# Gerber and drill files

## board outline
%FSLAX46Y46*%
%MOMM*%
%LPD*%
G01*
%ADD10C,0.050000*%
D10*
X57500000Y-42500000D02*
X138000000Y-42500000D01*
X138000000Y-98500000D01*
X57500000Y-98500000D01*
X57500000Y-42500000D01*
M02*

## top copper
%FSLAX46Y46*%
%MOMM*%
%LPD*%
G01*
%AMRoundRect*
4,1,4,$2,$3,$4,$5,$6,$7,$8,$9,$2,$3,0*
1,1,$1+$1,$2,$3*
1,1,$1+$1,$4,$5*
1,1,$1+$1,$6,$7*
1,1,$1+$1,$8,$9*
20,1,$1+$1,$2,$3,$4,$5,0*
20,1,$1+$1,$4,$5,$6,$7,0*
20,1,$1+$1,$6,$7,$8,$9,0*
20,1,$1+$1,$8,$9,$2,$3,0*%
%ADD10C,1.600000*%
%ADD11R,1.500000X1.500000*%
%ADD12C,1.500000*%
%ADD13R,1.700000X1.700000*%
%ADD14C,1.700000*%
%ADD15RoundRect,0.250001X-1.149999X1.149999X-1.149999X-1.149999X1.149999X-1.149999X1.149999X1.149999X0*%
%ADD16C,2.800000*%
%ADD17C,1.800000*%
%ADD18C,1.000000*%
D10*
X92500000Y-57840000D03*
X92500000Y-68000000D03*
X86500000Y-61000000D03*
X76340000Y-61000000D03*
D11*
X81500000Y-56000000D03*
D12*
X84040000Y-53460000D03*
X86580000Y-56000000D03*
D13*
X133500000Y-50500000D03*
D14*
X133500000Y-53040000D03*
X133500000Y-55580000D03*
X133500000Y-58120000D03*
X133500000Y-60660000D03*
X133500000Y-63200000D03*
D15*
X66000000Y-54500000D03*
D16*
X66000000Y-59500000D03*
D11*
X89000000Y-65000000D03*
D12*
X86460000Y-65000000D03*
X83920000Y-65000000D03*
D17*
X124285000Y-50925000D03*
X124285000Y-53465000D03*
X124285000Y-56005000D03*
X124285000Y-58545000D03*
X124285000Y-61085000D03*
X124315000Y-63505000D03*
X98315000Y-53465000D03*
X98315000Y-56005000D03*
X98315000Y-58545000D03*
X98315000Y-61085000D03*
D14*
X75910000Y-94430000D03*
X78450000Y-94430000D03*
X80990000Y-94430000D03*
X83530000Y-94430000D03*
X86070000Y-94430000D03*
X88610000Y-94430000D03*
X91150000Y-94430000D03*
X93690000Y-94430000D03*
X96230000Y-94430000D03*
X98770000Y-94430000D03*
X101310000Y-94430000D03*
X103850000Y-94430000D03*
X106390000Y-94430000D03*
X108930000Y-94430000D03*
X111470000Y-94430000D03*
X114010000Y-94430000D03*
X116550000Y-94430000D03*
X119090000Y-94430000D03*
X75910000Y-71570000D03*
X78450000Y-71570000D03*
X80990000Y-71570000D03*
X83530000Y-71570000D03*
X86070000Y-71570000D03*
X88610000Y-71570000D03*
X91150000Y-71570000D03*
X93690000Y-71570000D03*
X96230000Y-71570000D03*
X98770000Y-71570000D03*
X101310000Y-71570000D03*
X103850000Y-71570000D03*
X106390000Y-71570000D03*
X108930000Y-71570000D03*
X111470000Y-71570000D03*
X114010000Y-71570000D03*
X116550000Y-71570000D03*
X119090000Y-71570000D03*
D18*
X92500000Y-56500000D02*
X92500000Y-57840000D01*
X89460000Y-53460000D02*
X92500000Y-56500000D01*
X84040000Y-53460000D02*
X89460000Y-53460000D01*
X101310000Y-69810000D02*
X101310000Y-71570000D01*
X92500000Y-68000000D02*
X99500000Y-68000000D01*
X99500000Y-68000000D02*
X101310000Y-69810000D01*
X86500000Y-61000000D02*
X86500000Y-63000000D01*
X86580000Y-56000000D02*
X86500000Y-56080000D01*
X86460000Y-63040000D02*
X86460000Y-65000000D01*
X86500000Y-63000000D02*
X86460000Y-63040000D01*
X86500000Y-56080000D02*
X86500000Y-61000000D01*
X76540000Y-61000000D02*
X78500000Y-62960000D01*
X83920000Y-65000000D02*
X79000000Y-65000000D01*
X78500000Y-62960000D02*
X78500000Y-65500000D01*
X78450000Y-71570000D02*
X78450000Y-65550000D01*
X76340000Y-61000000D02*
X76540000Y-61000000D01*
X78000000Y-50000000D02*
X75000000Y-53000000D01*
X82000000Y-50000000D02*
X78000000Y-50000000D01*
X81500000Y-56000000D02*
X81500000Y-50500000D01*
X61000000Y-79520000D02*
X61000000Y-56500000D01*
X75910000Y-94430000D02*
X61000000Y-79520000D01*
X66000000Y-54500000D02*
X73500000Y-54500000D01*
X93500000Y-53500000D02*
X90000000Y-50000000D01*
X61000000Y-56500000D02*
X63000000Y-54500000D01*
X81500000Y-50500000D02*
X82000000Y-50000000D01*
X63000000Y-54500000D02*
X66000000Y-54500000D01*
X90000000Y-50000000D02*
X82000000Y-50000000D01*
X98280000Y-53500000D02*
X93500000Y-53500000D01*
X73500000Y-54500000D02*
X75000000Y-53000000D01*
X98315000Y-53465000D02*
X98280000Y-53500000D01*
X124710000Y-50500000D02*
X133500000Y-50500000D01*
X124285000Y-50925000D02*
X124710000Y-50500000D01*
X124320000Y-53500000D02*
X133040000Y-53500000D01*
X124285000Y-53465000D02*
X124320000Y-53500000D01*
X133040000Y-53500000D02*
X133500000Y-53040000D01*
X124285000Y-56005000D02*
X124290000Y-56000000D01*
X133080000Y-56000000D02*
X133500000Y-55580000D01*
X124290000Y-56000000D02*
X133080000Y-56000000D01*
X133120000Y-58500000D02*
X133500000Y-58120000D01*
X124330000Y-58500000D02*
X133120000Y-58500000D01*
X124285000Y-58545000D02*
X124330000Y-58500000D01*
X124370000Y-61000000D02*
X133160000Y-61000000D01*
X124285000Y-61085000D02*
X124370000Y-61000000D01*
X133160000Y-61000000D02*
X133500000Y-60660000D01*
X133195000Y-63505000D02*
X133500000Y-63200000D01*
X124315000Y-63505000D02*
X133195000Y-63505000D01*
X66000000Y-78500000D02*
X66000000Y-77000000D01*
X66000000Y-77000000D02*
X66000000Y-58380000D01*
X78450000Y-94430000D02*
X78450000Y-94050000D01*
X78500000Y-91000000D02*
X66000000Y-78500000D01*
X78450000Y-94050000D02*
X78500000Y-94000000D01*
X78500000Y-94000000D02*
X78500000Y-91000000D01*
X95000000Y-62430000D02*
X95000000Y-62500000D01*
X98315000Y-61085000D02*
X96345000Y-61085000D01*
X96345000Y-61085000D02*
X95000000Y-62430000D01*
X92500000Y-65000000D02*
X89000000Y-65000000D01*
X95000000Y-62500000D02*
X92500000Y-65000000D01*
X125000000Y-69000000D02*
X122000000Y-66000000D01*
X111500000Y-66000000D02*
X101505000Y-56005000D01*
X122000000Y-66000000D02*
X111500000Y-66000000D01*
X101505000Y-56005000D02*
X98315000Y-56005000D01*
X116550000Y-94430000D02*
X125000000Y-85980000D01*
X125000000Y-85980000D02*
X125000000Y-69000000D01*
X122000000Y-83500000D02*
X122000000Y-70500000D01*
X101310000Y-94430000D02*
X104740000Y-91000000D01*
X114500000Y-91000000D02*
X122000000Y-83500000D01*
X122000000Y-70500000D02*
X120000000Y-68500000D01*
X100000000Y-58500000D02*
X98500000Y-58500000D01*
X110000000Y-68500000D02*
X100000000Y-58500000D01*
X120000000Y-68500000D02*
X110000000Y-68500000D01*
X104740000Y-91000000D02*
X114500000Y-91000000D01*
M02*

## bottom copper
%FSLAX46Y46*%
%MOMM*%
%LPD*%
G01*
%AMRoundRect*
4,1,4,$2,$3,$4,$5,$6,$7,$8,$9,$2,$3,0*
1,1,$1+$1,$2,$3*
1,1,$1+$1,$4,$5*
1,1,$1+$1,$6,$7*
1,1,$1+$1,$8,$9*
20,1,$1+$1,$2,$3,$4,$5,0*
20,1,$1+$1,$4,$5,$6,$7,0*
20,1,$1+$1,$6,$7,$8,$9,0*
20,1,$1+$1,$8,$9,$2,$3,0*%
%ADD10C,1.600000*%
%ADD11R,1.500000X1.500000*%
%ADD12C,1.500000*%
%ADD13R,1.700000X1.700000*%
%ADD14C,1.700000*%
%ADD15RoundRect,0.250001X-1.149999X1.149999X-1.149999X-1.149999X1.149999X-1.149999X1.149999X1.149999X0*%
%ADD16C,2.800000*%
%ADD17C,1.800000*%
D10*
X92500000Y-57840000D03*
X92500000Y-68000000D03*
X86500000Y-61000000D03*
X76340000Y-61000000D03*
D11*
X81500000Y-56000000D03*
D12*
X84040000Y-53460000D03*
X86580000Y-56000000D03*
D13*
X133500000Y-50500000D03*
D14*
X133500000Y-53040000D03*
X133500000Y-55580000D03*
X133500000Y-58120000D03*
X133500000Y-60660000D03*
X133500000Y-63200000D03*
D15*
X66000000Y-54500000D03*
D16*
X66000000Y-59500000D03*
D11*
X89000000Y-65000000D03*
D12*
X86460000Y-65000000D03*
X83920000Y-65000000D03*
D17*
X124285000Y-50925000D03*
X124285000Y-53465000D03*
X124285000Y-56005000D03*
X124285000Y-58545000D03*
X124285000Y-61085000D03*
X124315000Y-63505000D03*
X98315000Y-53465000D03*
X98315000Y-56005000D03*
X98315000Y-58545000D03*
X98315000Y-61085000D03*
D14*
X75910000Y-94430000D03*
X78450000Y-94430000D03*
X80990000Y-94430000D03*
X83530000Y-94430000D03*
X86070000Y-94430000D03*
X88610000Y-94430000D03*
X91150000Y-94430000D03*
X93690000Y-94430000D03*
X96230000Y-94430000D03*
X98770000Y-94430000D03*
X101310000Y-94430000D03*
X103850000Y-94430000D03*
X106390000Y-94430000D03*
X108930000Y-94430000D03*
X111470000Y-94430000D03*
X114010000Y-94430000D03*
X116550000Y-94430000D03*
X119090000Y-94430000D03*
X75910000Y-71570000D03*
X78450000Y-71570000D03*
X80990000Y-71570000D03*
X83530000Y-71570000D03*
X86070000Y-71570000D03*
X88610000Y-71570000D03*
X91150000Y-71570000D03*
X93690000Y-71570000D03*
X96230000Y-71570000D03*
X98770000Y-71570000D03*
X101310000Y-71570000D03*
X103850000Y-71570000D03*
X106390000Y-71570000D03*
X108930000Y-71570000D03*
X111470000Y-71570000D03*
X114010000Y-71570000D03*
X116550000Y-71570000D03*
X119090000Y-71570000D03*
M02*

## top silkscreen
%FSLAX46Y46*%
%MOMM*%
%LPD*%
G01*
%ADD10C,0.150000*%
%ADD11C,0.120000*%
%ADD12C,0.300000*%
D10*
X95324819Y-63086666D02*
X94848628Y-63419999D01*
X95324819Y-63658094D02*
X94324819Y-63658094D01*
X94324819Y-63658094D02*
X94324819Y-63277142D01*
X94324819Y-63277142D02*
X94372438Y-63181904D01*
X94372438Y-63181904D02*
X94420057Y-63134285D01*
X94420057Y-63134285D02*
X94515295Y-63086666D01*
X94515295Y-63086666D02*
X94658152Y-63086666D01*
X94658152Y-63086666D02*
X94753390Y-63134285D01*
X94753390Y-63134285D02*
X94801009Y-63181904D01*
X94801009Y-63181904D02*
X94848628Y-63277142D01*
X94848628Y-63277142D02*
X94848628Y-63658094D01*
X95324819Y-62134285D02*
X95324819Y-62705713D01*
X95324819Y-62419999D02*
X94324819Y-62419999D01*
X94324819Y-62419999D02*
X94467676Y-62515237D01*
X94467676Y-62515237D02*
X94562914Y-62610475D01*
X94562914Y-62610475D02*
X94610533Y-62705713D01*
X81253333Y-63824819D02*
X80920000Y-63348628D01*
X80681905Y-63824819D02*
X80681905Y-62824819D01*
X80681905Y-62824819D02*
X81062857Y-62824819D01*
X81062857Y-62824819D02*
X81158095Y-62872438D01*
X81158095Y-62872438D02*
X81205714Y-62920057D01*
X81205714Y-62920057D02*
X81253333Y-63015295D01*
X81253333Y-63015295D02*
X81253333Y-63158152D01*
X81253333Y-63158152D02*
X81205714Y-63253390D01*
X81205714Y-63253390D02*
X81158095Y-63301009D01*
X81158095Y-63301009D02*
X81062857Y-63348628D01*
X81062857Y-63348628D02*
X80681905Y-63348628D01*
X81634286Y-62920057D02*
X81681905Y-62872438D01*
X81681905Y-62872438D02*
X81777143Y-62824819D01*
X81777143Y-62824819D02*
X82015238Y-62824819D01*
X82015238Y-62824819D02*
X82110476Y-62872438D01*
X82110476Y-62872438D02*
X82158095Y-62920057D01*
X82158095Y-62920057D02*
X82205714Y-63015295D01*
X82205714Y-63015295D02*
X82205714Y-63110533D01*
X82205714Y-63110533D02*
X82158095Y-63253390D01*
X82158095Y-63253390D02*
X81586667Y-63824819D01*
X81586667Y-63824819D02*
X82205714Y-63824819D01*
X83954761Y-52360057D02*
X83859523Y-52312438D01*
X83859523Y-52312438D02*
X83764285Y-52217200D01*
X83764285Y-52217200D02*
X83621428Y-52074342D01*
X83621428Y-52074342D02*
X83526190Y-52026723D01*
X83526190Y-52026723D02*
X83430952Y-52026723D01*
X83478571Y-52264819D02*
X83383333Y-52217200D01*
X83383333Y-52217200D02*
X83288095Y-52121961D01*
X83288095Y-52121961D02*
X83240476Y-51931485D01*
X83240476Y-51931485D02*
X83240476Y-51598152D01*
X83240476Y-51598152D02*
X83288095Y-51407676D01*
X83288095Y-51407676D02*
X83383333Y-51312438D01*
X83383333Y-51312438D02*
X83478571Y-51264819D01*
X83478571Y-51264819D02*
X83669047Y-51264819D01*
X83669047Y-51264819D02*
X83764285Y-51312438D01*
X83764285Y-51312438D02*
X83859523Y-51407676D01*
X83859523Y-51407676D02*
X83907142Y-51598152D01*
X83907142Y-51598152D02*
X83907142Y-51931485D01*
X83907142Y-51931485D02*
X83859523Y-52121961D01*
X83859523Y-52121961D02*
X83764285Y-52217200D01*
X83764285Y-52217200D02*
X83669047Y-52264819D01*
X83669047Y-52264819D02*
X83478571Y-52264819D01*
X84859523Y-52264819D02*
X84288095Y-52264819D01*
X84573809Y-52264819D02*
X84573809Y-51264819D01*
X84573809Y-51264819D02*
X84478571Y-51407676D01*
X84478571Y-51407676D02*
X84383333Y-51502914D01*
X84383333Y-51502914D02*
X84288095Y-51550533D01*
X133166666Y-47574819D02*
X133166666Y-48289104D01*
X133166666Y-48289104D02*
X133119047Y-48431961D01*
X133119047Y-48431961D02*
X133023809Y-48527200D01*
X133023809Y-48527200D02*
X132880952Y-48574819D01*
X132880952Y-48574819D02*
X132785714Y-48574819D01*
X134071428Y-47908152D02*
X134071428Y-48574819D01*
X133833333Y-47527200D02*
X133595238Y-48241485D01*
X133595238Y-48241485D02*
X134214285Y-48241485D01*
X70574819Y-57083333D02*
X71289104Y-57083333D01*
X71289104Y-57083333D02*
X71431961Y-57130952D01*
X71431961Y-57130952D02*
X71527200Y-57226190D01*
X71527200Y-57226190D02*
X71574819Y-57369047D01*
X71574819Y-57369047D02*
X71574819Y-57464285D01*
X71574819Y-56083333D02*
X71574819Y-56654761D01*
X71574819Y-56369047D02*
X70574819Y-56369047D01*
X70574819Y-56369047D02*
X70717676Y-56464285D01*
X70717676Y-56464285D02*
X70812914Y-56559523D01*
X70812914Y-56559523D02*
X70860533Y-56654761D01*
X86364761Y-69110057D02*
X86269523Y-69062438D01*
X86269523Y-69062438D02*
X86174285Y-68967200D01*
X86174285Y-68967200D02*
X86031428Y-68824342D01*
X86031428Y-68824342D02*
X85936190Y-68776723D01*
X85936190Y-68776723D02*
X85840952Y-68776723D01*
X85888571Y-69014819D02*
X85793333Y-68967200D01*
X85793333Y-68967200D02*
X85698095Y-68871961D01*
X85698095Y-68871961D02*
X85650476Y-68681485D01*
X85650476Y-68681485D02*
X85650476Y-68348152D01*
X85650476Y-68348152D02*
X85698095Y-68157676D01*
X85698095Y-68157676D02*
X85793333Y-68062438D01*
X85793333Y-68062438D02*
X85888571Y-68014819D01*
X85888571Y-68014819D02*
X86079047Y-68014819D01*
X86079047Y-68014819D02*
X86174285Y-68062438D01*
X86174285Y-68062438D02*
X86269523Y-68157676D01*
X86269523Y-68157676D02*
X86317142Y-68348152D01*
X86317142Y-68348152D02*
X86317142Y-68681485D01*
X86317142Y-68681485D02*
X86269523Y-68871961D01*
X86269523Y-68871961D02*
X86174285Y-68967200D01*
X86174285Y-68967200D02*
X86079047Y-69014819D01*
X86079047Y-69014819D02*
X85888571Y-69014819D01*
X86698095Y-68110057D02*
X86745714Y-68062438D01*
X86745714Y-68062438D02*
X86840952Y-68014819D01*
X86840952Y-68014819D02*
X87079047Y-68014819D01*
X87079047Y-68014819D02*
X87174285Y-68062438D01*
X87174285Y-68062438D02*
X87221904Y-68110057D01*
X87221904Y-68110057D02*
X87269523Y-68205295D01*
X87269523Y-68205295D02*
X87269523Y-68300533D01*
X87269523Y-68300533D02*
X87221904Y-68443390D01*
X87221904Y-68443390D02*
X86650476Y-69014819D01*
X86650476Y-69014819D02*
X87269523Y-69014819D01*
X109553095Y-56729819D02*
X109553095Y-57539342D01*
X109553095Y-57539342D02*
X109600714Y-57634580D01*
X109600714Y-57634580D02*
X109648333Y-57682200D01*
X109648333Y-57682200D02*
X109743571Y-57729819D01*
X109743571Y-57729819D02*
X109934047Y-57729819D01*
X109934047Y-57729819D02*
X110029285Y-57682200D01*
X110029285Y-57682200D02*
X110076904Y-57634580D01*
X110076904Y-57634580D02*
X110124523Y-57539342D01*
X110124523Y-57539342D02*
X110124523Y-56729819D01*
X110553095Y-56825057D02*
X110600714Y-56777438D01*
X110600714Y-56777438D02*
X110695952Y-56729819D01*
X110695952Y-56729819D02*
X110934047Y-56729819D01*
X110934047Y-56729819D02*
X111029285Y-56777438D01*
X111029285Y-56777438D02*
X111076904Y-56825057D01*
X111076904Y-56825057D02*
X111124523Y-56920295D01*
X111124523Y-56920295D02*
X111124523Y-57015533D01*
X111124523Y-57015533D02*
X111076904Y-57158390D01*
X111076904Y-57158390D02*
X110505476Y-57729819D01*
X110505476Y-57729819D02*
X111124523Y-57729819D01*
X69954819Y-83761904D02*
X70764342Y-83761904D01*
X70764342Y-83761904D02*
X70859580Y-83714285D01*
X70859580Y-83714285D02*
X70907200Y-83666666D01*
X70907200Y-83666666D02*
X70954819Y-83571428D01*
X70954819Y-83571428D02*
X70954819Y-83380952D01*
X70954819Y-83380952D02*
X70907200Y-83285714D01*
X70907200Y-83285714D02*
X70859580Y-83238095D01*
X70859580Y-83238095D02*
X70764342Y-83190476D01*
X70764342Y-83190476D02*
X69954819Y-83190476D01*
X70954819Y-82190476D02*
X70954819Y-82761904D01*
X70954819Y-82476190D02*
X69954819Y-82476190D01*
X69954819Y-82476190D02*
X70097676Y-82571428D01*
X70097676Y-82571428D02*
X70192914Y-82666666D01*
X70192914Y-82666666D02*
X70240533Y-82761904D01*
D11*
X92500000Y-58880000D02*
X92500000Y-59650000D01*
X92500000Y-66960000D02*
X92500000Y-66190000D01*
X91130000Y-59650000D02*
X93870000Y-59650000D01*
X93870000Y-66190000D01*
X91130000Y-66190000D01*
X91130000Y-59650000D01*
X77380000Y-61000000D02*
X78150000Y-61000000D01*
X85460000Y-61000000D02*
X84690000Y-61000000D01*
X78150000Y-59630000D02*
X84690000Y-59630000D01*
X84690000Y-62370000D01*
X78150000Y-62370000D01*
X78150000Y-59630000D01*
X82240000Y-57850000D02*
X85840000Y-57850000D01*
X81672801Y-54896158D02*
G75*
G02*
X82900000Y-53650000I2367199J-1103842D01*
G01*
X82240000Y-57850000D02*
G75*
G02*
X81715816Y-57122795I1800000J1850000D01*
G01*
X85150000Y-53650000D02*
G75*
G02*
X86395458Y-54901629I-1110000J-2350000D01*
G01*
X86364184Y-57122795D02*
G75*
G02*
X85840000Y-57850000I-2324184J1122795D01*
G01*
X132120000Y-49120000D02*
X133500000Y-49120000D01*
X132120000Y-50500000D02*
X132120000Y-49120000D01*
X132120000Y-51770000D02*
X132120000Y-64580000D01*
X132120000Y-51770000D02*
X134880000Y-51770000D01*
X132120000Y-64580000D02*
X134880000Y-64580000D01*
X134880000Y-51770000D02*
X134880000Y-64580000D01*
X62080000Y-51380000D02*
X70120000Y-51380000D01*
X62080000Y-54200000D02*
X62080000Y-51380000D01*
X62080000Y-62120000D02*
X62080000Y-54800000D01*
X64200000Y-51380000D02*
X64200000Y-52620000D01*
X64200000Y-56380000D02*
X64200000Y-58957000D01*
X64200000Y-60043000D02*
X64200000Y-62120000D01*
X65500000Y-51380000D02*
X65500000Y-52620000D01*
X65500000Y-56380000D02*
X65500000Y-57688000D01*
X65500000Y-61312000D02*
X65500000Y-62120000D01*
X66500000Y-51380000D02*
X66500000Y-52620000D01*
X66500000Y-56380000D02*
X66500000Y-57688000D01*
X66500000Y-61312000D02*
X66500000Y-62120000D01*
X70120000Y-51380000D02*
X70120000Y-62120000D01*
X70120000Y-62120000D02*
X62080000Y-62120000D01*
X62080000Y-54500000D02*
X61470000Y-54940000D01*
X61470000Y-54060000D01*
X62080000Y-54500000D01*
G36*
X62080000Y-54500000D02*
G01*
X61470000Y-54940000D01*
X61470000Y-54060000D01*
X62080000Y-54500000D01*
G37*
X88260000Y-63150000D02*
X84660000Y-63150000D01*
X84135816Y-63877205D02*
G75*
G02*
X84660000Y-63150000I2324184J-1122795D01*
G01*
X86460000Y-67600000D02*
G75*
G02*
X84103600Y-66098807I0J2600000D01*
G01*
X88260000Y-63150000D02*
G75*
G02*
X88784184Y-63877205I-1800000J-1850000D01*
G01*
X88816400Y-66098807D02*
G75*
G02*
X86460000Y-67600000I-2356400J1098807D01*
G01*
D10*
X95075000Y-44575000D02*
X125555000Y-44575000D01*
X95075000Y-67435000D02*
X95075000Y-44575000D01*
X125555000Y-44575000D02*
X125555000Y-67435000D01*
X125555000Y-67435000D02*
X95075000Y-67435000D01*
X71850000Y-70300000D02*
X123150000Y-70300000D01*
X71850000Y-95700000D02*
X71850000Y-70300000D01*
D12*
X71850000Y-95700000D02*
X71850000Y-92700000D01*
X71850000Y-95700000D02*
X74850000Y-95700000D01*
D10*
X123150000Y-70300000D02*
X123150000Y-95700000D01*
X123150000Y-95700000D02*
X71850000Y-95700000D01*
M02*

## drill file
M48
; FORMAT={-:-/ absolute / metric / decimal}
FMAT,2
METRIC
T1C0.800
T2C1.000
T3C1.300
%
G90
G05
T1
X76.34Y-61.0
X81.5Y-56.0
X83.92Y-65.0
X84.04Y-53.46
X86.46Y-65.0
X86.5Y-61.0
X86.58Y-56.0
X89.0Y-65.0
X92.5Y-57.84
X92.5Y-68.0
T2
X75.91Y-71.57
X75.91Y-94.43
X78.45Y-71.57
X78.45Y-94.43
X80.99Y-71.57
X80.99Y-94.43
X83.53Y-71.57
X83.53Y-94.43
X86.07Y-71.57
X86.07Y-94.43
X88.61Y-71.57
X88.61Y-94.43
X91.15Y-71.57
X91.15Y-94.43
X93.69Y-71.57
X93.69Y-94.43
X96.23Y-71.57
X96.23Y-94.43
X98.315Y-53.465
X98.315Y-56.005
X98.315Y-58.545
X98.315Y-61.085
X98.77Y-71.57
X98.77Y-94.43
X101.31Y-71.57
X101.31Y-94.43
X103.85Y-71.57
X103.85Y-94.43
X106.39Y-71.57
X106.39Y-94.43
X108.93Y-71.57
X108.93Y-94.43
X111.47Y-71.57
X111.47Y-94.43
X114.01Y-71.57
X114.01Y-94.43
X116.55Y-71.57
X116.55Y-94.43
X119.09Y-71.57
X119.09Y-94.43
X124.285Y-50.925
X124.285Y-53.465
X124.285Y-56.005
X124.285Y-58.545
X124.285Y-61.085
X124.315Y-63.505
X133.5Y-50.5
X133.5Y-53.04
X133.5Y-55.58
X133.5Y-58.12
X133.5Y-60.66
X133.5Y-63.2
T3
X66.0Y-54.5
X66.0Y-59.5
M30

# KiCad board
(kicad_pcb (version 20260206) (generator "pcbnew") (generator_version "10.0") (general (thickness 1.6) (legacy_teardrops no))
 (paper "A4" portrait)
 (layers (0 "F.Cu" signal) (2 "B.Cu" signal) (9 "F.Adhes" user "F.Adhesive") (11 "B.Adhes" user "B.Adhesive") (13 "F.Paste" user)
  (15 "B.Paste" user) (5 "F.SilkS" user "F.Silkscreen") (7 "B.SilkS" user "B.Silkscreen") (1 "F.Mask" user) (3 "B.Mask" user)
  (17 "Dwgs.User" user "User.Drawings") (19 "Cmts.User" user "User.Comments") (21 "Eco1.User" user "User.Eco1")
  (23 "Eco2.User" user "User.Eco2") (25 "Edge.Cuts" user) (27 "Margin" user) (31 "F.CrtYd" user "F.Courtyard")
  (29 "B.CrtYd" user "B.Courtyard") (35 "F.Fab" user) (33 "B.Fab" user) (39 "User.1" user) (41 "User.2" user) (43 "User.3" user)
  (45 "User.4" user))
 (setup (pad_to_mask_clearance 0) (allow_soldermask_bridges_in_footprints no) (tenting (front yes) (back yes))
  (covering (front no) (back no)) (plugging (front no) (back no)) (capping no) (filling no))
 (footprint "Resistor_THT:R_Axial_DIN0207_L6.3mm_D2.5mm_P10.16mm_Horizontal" (layer "F.Cu") (at 92.5 57.84 -90)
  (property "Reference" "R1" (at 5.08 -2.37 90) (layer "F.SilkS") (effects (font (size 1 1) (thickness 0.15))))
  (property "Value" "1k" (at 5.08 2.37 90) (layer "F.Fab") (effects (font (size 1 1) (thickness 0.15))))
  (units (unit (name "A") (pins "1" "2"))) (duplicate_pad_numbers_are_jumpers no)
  (fp_line (start 1.04 0) (end 1.81 0) (stroke (width 0.12) (type solid)) (layer "F.SilkS"))
  (fp_line (start 9.12 0) (end 8.35 0) (stroke (width 0.12) (type solid)) (layer "F.SilkS"))
  (fp_rect (start 1.81 -1.37) (end 8.35 1.37) (stroke (width 0.12) (type solid)) (fill no) (layer "F.SilkS"))
  (pad "1" thru_hole circle (at 0 0 270) (size 1.6 1.6) (drill 0.8) (layers "*.Cu" "*.Mask") (remove_unused_layers no) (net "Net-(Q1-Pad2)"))
  (pad "2" thru_hole circle (at 10.16 0 270) (size 1.6 1.6) (drill 0.8) (layers "*.Cu" "*.Mask") (remove_unused_layers no)
   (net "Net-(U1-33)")))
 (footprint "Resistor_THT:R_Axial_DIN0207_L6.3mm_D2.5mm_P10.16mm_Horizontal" (layer "F.Cu") (at 86.5 61 180)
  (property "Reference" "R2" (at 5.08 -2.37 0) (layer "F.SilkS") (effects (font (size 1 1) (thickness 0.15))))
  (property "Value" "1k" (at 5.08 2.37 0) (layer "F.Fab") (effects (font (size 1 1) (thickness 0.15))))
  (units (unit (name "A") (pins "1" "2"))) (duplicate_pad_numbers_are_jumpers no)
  (fp_line (start 9.12 0) (end 8.35 0) (stroke (width 0.12) (type solid)) (layer "F.SilkS"))
  (fp_line (start 1.04 0) (end 1.81 0) (stroke (width 0.12) (type solid)) (layer "F.SilkS"))
  (fp_rect (start 1.81 -1.37) (end 8.35 1.37) (stroke (width 0.12) (type solid)) (fill no) (layer "F.SilkS"))
  (pad "1" thru_hole circle (at 0 0 180) (size 1.6 1.6) (drill 0.8) (layers "*.Cu" "*.Mask") (remove_unused_layers no) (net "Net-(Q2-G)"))
  (pad "2" thru_hole circle (at 10.16 0 180) (size 1.6 1.6) (drill 0.8) (layers "*.Cu" "*.Mask") (remove_unused_layers no)
   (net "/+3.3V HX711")))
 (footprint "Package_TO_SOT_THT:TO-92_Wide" (layer "F.Cu") (at 81.5 56)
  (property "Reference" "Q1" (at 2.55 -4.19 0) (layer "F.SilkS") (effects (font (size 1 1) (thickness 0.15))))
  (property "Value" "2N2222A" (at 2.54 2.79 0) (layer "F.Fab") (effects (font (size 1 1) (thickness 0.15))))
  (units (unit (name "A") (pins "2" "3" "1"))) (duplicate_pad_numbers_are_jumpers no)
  (fp_line (start 0.74 1.85) (end 4.34 1.85) (stroke (width 0.12) (type solid)) (layer "F.SilkS"))
  (fp_arc (start 0.172801 -1.103842) (mid 0.678995 -1.832692) (end 1.4 -2.35) (stroke (width 0.12) (type solid)) (layer "F.SilkS"))
  (fp_arc (start 0.74 1.85) (mid 0.446097 1.509328) (end 0.215816 1.122795) (stroke (width 0.12) (type solid)) (layer "F.SilkS"))
  (fp_arc (start 3.65 -2.35) (mid 4.382279 -1.833196) (end 4.895458 -1.098371) (stroke (width 0.12) (type solid)) (layer "F.SilkS"))
  (fp_arc (start 4.864184 1.122795) (mid 4.633903 1.509328) (end 4.34 1.85) (stroke (width 0.12) (type solid)) (layer "F.SilkS"))
  (pad "1" thru_hole rect (at 0 0) (size 1.5 1.5) (drill 0.8) (layers "*.Cu" "*.Mask") (remove_unused_layers no) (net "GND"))
  (pad "2" thru_hole circle (at 2.54 -2.54) (size 1.5 1.5) (drill 0.8) (layers "*.Cu" "*.Mask") (remove_unused_layers no)
   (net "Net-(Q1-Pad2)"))
  (pad "3" thru_hole circle (at 5.08 0) (size 1.5 1.5) (drill 0.8) (layers "*.Cu" "*.Mask") (remove_unused_layers no) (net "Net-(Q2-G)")))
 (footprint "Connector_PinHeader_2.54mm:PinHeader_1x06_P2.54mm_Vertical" (layer "F.Cu") (at 133.5 50.5)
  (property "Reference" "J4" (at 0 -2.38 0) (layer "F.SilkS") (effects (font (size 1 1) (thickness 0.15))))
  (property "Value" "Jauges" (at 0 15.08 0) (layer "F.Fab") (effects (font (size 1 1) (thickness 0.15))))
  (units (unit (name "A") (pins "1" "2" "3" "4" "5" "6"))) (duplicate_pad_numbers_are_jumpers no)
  (fp_line (start -1.38 -1.38) (end 0 -1.38) (stroke (width 0.12) (type solid)) (layer "F.SilkS"))
  (fp_line (start -1.38 0) (end -1.38 -1.38) (stroke (width 0.12) (type solid)) (layer "F.SilkS"))
  (fp_line (start -1.38 1.27) (end -1.38 14.08) (stroke (width 0.12) (type solid)) (layer "F.SilkS"))
  (fp_line (start -1.38 1.27) (end 1.38 1.27) (stroke (width 0.12) (type solid)) (layer "F.SilkS"))
  (fp_line (start -1.38 14.08) (end 1.38 14.08) (stroke (width 0.12) (type solid)) (layer "F.SilkS"))
  (fp_line (start 1.38 1.27) (end 1.38 14.08) (stroke (width 0.12) (type solid)) (layer "F.SilkS"))
  (pad "1" thru_hole rect (at 0 0) (size 1.7 1.7) (drill 1) (layers "*.Cu" "*.Mask") (remove_unused_layers no) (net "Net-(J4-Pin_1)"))
  (pad "2" thru_hole circle (at 0 2.54) (size 1.7 1.7) (drill 1) (layers "*.Cu" "*.Mask") (remove_unused_layers no) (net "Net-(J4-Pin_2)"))
  (pad "3" thru_hole circle (at 0 5.08) (size 1.7 1.7) (drill 1) (layers "*.Cu" "*.Mask") (remove_unused_layers no) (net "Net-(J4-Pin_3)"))
  (pad "4" thru_hole circle (at 0 7.62) (size 1.7 1.7) (drill 1) (layers "*.Cu" "*.Mask") (remove_unused_layers no) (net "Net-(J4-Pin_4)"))
  (pad "5" thru_hole circle (at 0 10.16) (size 1.7 1.7) (drill 1) (layers "*.Cu" "*.Mask") (remove_unused_layers no) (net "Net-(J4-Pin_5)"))
  (pad "6" thru_hole circle (at 0 12.7) (size 1.7 1.7) (drill 1) (layers "*.Cu" "*.Mask") (remove_unused_layers no) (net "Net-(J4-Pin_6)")))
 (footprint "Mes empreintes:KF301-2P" (layer "F.Cu") (at 66 54.5 -90)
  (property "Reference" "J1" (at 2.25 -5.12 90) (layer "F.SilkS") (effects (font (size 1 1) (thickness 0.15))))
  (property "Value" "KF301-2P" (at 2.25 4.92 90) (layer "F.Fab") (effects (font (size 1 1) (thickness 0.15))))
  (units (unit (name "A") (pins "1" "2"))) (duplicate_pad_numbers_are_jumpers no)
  (fp_line (start -3.12 3.92) (end -3.12 -4.12) (stroke (width 0.12) (type solid)) (layer "F.SilkS"))
  (fp_line (start -0.3 3.92) (end -3.12 3.92) (stroke (width 0.12) (type solid)) (layer "F.SilkS"))
  (fp_line (start 7.62 3.92) (end 0.3 3.92) (stroke (width 0.12) (type solid)) (layer "F.SilkS"))
  (fp_line (start -3.12 1.8) (end -1.88 1.8) (stroke (width 0.12) (type solid)) (layer "F.SilkS"))
  (fp_line (start 1.88 1.8) (end 4.457 1.8) (stroke (width 0.12) (type solid)) (layer "F.SilkS"))
  (fp_line (start 5.543 1.8) (end 7.62 1.8) (stroke (width 0.12) (type solid)) (layer "F.SilkS"))
  (fp_line (start -3.12 0.5) (end -1.88 0.5) (stroke (width 0.12) (type solid)) (layer "F.SilkS"))
  (fp_line (start 1.88 0.5) (end 3.188 0.5) (stroke (width 0.12) (type solid)) (layer "F.SilkS"))
  (fp_line (start 6.812 0.5) (end 7.62 0.5) (stroke (width 0.12) (type solid)) (layer "F.SilkS"))
  (fp_line (start -3.12 -0.5) (end -1.88 -0.5) (stroke (width 0.12) (type solid)) (layer "F.SilkS"))
  (fp_line (start 1.88 -0.5) (end 3.188 -0.5) (stroke (width 0.12) (type solid)) (layer "F.SilkS"))
  (fp_line (start 6.812 -0.5) (end 7.62 -0.5) (stroke (width 0.12) (type solid)) (layer "F.SilkS"))
  (fp_line (start -3.12 -4.12) (end 7.62 -4.12) (stroke (width 0.12) (type solid)) (layer "F.SilkS"))
  (fp_line (start 7.62 -4.12) (end 7.62 3.92) (stroke (width 0.12) (type solid)) (layer "F.SilkS"))
  (fp_poly (pts (xy 0 3.92) (xy 0.44 4.53) (xy -0.44 4.53)) (stroke (width 0.12) (type solid)) (fill yes) (layer "F.SilkS"))
  (pad "1" thru_hole roundrect (at 0 0 270) (size 2.8 2.8) (drill 1.3) (layers "*.Cu" "*.Mask") (remove_unused_layers no)
   (roundrect_rratio 0.089286) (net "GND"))
  (pad "2" thru_hole circle (at 5 0 270) (size 2.8 2.8) (drill 1.3) (layers "*.Cu" "*.Mask") (remove_unused_layers no) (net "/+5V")))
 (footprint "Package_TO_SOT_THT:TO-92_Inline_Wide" (layer "F.Cu") (at 89 65 180)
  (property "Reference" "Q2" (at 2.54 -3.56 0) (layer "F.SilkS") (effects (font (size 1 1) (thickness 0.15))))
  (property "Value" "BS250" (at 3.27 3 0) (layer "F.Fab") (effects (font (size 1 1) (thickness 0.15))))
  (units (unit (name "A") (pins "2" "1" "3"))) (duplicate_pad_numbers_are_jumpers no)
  (fp_line (start 0.74 1.85) (end 4.34 1.85) (stroke (width 0.12) (type solid)) (layer "F.SilkS"))
  (fp_arc (start 4.864184 1.122795) (mid 4.633903 1.509328) (end 4.34 1.85) (stroke (width 0.12) (type solid)) (layer "F.SilkS"))
  (fp_arc (start 2.54 -2.6) (mid 3.936979 -2.192818) (end 4.8964 -1.098807) (stroke (width 0.12) (type solid)) (layer "F.SilkS"))
  (fp_arc (start 0.74 1.85) (mid 0.446097 1.509328) (end 0.215816 1.122795) (stroke (width 0.12) (type solid)) (layer "F.SilkS"))
  (fp_arc (start 0.1836 -1.098807) (mid 1.143021 -2.192817) (end 2.54 -2.6) (stroke (width 0.12) (type solid)) (layer "F.SilkS"))
  (pad "1" thru_hole rect (at 0 0 180) (size 1.5 1.5) (drill 0.8) (layers "*.Cu" "*.Mask") (remove_unused_layers no) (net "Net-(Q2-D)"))
  (pad "2" thru_hole circle (at 2.54 0 180) (size 1.5 1.5) (drill 0.8) (layers "*.Cu" "*.Mask") (remove_unused_layers no) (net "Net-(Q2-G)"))
  (pad "3" thru_hole circle (at 5.08 0 180) (size 1.5 1.5) (drill 0.8) (layers "*.Cu" "*.Mask") (remove_unused_layers no)
   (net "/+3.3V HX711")))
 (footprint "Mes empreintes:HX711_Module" (layer "F.Cu") (at 110.315 56.005)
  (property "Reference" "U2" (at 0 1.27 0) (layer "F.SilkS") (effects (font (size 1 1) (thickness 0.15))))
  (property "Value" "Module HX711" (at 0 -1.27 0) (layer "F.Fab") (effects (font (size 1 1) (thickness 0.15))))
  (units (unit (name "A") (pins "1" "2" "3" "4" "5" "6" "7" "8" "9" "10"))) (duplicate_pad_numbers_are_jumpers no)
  (fp_line (start -15.24 -11.43) (end 15.24 -11.43) (stroke (width 0.15) (type solid)) (layer "F.SilkS"))
  (fp_line (start -15.24 11.43) (end -15.24 -11.43) (stroke (width 0.15) (type solid)) (layer "F.SilkS"))
  (fp_line (start 15.24 -11.43) (end 15.24 11.43) (stroke (width 0.15) (type solid)) (layer "F.SilkS"))
  (fp_line (start 15.24 11.43) (end -15.24 11.43) (stroke (width 0.15) (type solid)) (layer "F.SilkS"))
  (pad "1" thru_hole circle (at 13.97 -5.08) (size 1.8 1.8) (drill 1) (layers "*.Cu" "*.Mask") (remove_unused_layers no)
   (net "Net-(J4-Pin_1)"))
  (pad "2" thru_hole circle (at 13.97 -2.54) (size 1.8 1.8) (drill 1) (layers "*.Cu" "*.Mask") (remove_unused_layers no)
   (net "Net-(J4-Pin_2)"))
  (pad "3" thru_hole circle (at 13.97 0) (size 1.8 1.8) (drill 1) (layers "*.Cu" "*.Mask") (remove_unused_layers no) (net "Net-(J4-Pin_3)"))
  (pad "4" thru_hole circle (at 13.97 2.54) (size 1.8 1.8) (drill 1) (layers "*.Cu" "*.Mask") (remove_unused_layers no)
   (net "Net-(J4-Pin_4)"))
  (pad "5" thru_hole circle (at 13.97 5.08) (size 1.8 1.8) (drill 1) (layers "*.Cu" "*.Mask") (remove_unused_layers no)
   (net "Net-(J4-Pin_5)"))
  (pad "6" thru_hole circle (at 14 7.5) (size 1.8 1.8) (drill 1) (layers "*.Cu" "*.Mask") (remove_unused_layers no) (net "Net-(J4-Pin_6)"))
  (pad "7" thru_hole circle (at -12 -2.54) (size 1.8 1.8) (drill 1) (layers "*.Cu" "*.Mask") (remove_unused_layers no) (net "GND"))
  (pad "8" thru_hole circle (at -12 0) (size 1.8 1.8) (drill 1) (layers "*.Cu" "*.Mask") (remove_unused_layers no) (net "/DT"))
  (pad "9" thru_hole circle (at -12 2.54) (size 1.8 1.8) (drill 1) (layers "*.Cu" "*.Mask") (remove_unused_layers no) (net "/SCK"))
  (pad "10" thru_hole circle (at -12 5.08) (size 1.8 1.8) (drill 1) (layers "*.Cu" "*.Mask") (remove_unused_layers no) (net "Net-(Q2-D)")))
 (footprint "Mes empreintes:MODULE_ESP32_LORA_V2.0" (layer "F.Cu") (at 97.5 83 90)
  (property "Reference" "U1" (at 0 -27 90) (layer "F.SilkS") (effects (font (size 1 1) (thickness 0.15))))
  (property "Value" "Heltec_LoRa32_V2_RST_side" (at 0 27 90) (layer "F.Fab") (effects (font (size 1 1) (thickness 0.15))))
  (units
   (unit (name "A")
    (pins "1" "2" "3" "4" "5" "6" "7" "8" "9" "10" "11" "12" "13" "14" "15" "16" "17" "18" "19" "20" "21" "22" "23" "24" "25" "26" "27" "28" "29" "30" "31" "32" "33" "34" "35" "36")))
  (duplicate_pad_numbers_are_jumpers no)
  (fp_line (start 12.7 -25.65) (end 12.7 25.65) (stroke (width 0.15) (type solid)) (layer "F.SilkS"))
  (fp_line (start -12.7 -25.65) (end 12.7 -25.65) (stroke (width 0.15) (type solid)) (layer "F.SilkS"))
  (fp_line (start -12.7 -25.65) (end -9.7 -25.65) (stroke (width 0.3) (type solid)) (layer "F.SilkS"))
  (fp_line (start -12.7 -25.65) (end -12.7 -22.65) (stroke (width 0.3) (type solid)) (layer "F.SilkS"))
  (fp_line (start 12.7 25.65) (end -12.7 25.65) (stroke (width 0.15) (type solid)) (layer "F.SilkS"))
  (fp_line (start -12.7 25.65) (end -12.7 -25.65) (stroke (width 0.15) (type solid)) (layer "F.SilkS"))
  (pad "1" thru_hole circle (at -11.43 -21.59 90) (size 1.7 1.7) (drill 1) (layers "*.Cu" "*.Mask") (remove_unused_layers no) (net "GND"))
  (pad "2" thru_hole circle (at -11.43 -19.05 90) (size 1.7 1.7) (drill 1) (layers "*.Cu" "*.Mask") (remove_unused_layers no) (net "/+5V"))
  (pad "3" thru_hole circle (at -11.43 -16.51 90) (size 1.7 1.7) (drill 1) (layers "*.Cu" "*.Mask") (remove_unused_layers no)
   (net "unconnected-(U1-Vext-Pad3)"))
  (pad "4" thru_hole circle (at -11.43 -13.97 90) (size 1.7 1.7) (drill 1) (layers "*.Cu" "*.Mask") (remove_unused_layers no)
   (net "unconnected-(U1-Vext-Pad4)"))
  (pad "5" thru_hole circle (at -11.43 -11.43 90) (size 1.7 1.7) (drill 1) (layers "*.Cu" "*.Mask") (remove_unused_layers no)
   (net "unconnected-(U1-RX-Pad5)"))
  (pad "6" thru_hole circle (at -11.43 -8.89 90) (size 1.7 1.7) (drill 1) (layers "*.Cu" "*.Mask") (remove_unused_layers no)
   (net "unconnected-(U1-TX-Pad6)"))
  (pad "7" thru_hole circle (at -11.43 -6.35 90) (size 1.7 1.7) (drill 1) (layers "*.Cu" "*.Mask") (remove_unused_layers no)
   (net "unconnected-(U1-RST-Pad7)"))
  (pad "8" thru_hole circle (at -11.43 -3.81 90) (size 1.7 1.7) (drill 1) (layers "*.Cu" "*.Mask") (remove_unused_layers no)
   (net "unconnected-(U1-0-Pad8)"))
  (pad "9" thru_hole circle (at -11.43 -1.27 90) (size 1.7 1.7) (drill 1) (layers "*.Cu" "*.Mask") (remove_unused_layers no)
   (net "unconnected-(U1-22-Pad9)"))
  (pad "10" thru_hole circle (at -11.43 1.27 90) (size 1.7 1.7) (drill 1) (layers "*.Cu" "*.Mask") (remove_unused_layers no)
   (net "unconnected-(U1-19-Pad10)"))
  (pad "11" thru_hole circle (at -11.43 3.81 90) (size 1.7 1.7) (drill 1) (layers "*.Cu" "*.Mask") (remove_unused_layers no) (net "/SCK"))
  (pad "12" thru_hole circle (at -11.43 6.35 90) (size 1.7 1.7) (drill 1) (layers "*.Cu" "*.Mask") (remove_unused_layers no)
   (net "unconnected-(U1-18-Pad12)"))
  (pad "13" thru_hole circle (at -11.43 8.89 90) (size 1.7 1.7) (drill 1) (layers "*.Cu" "*.Mask") (remove_unused_layers no)
   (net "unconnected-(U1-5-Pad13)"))
  (pad "14" thru_hole circle (at -11.43 11.43 90) (size 1.7 1.7) (drill 1) (layers "*.Cu" "*.Mask") (remove_unused_layers no)
   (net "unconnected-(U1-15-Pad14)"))
  (pad "15" thru_hole circle (at -11.43 13.97 90) (size 1.7 1.7) (drill 1) (layers "*.Cu" "*.Mask") (remove_unused_layers no)
   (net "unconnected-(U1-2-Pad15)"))
  (pad "16" thru_hole circle (at -11.43 16.51 90) (size 1.7 1.7) (drill 1) (layers "*.Cu" "*.Mask") (remove_unused_layers no)
   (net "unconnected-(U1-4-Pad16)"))
  (pad "17" thru_hole circle (at -11.43 19.05 90) (size 1.7 1.7) (drill 1) (layers "*.Cu" "*.Mask") (remove_unused_layers no) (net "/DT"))
  (pad "18" thru_hole circle (at -11.43 21.59 90) (size 1.7 1.7) (drill 1) (layers "*.Cu" "*.Mask") (remove_unused_layers no)
   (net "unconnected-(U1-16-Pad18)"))
  (pad "19" thru_hole circle (at 11.43 -21.59 90) (size 1.7 1.7) (drill 1) (layers "*.Cu" "*.Mask") (remove_unused_layers no)
   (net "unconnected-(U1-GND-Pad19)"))
  (pad "20" thru_hole circle (at 11.43 -19.05 90) (size 1.7 1.7) (drill 1) (layers "*.Cu" "*.Mask") (remove_unused_layers no)
   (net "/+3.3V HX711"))
  (pad "21" thru_hole circle (at 11.43 -16.51 90) (size 1.7 1.7) (drill 1) (layers "*.Cu" "*.Mask") (remove_unused_layers no)
   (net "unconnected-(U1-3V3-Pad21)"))
  (pad "22" thru_hole circle (at 11.43 -13.97 90) (size 1.7 1.7) (drill 1) (layers "*.Cu" "*.Mask") (remove_unused_layers no)
   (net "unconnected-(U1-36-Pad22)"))
  (pad "23" thru_hole circle (at 11.43 -11.43 90) (size 1.7 1.7) (drill 1) (layers "*.Cu" "*.Mask") (remove_unused_layers no)
   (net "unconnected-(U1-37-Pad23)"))
  (pad "24" thru_hole circle (at 11.43 -8.89 90) (size 1.7 1.7) (drill 1) (layers "*.Cu" "*.Mask") (remove_unused_layers no)
   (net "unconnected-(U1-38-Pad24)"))
  (pad "25" thru_hole circle (at 11.43 -6.35 90) (size 1.7 1.7) (drill 1) (layers "*.Cu" "*.Mask") (remove_unused_layers no)
   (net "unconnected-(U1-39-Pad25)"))
  (pad "26" thru_hole circle (at 11.43 -3.81 90) (size 1.7 1.7) (drill 1) (layers "*.Cu" "*.Mask") (remove_unused_layers no)
   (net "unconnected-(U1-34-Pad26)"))
  (pad "27" thru_hole circle (at 11.43 -1.27 90) (size 1.7 1.7) (drill 1) (layers "*.Cu" "*.Mask") (remove_unused_layers no)
   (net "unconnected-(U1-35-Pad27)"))
  (pad "28" thru_hole circle (at 11.43 1.27 90) (size 1.7 1.7) (drill 1) (layers "*.Cu" "*.Mask") (remove_unused_layers no)
   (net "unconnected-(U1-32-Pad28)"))
  (pad "29" thru_hole circle (at 11.43 3.81 90) (size 1.7 1.7) (drill 1) (layers "*.Cu" "*.Mask") (remove_unused_layers no)
   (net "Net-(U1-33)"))
  (pad "30" thru_hole circle (at 11.43 6.35 90) (size 1.7 1.7) (drill 1) (layers "*.Cu" "*.Mask") (remove_unused_layers no)
   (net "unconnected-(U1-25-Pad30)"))
  (pad "31" thru_hole circle (at 11.43 8.89 90) (size 1.7 1.7) (drill 1) (layers "*.Cu" "*.Mask") (remove_unused_layers no)
   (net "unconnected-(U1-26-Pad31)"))
  (pad "32" thru_hole circle (at 11.43 11.43 90) (size 1.7 1.7) (drill 1) (layers "*.Cu" "*.Mask") (remove_unused_layers no)
   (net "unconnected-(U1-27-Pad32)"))
  (pad "33" thru_hole circle (at 11.43 13.97 90) (size 1.7 1.7) (drill 1) (layers "*.Cu" "*.Mask") (remove_unused_layers no)
   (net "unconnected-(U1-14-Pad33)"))
  (pad "34" thru_hole circle (at 11.43 16.51 90) (size 1.7 1.7) (drill 1) (layers "*.Cu" "*.Mask") (remove_unused_layers no)
   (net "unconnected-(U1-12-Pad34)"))
  (pad "35" thru_hole circle (at 11.43 19.05 90) (size 1.7 1.7) (drill 1) (layers "*.Cu" "*.Mask") (remove_unused_layers no)
   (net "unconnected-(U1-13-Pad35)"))
  (pad "36" thru_hole circle (at 11.43 21.59 90) (size 1.7 1.7) (drill 1) (layers "*.Cu" "*.Mask") (remove_unused_layers no)
   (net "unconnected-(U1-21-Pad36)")))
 (gr_rect (start 57.5 42.5) (end 138 98.5) (stroke (width 0.05) (type solid)) (fill no) (layer "Edge.Cuts"))
 (segment (start 92.5 56.5) (end 92.5 57.84) (width 1) (layer "F.Cu") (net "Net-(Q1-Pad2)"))
 (segment (start 89.46 53.46) (end 92.5 56.5) (width 1) (layer "F.Cu") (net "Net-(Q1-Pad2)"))
 (segment (start 84.04 53.46) (end 89.46 53.46) (width 1) (layer "F.Cu") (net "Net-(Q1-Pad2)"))
 (segment (start 101.31 69.81) (end 101.31 71.57) (width 1) (layer "F.Cu") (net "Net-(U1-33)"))
 (segment (start 92.5 68) (end 99.5 68) (width 1) (layer "F.Cu") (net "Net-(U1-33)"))
 (segment (start 99.5 68) (end 101.31 69.81) (width 1) (layer "F.Cu") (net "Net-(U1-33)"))
 (segment (start 86.5 61) (end 86.5 63) (width 1) (layer "F.Cu") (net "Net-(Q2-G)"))
 (segment (start 86.58 56) (end 86.5 56.08) (width 1) (layer "F.Cu") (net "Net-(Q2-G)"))
 (segment (start 86.46 63.04) (end 86.46 65) (width 1) (layer "F.Cu") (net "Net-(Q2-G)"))
 (segment (start 86.5 63) (end 86.46 63.04) (width 1) (layer "F.Cu") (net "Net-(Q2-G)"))
 (segment (start 86.5 56.08) (end 86.5 61) (width 1) (layer "F.Cu") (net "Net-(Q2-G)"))
 (segment (start 76.54 61) (end 78.5 62.96) (width 1) (layer "F.Cu") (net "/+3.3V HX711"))
 (segment (start 83.92 65) (end 79 65) (width 1) (layer "F.Cu") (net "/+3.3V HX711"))
 (segment (start 78.5 62.96) (end 78.5 65.5) (width 1) (layer "F.Cu") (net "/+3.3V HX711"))
 (segment (start 78.45 71.57) (end 78.45 65.55) (width 1) (layer "F.Cu") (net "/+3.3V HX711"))
 (segment (start 76.34 61) (end 76.54 61) (width 1) (layer "F.Cu") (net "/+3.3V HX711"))
 (segment (start 78 50) (end 75 53) (width 1) (layer "F.Cu") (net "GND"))
 (segment (start 82 50) (end 78 50) (width 1) (layer "F.Cu") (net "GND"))
 (segment (start 81.5 56) (end 81.5 50.5) (width 1) (layer "F.Cu") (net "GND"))
 (segment (start 61 79.52) (end 61 56.5) (width 1) (layer "F.Cu") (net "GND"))
 (segment (start 75.91 94.43) (end 61 79.52) (width 1) (layer "F.Cu") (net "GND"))
 (segment (start 66 54.5) (end 73.5 54.5) (width 1) (layer "F.Cu") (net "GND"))
 (segment (start 93.5 53.5) (end 90 50) (width 1) (layer "F.Cu") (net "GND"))
 (segment (start 61 56.5) (end 63 54.5) (width 1) (layer "F.Cu") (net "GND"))
 (segment (start 81.5 50.5) (end 82 50) (width 1) (layer "F.Cu") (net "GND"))
 (segment (start 63 54.5) (end 66 54.5) (width 1) (layer "F.Cu") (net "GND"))
 (segment (start 90 50) (end 82 50) (width 1) (layer "F.Cu") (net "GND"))
 (segment (start 98.28 53.5) (end 93.5 53.5) (width 1) (layer "F.Cu") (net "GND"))
 (segment (start 73.5 54.5) (end 75 53) (width 1) (layer "F.Cu") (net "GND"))
 (segment (start 98.315 53.465) (end 98.28 53.5) (width 1) (layer "F.Cu") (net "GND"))
 (segment (start 124.71 50.5) (end 133.5 50.5) (width 1) (layer "F.Cu") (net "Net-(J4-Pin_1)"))
 (segment (start 124.285 50.925) (end 124.71 50.5) (width 1) (layer "F.Cu") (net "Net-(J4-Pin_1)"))
 (segment (start 124.32 53.5) (end 133.04 53.5) (width 1) (layer "F.Cu") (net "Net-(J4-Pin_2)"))
 (segment (start 124.285 53.465) (end 124.32 53.5) (width 1) (layer "F.Cu") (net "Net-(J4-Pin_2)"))
 (segment (start 133.04 53.5) (end 133.5 53.04) (width 1) (layer "F.Cu") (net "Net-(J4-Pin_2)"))
 (segment (start 124.285 56.005) (end 124.29 56) (width 1) (layer "F.Cu") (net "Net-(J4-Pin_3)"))
 (segment (start 133.08 56) (end 133.5 55.58) (width 1) (layer "F.Cu") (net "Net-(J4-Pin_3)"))
 (segment (start 124.29 56) (end 133.08 56) (width 1) (layer "F.Cu") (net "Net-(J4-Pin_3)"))
 (segment (start 133.12 58.5) (end 133.5 58.12) (width 1) (layer "F.Cu") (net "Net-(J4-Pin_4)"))
 (segment (start 124.33 58.5) (end 133.12 58.5) (width 1) (layer "F.Cu") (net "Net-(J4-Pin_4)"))
 (segment (start 124.285 58.545) (end 124.33 58.5) (width 1) (layer "F.Cu") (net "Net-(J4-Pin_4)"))
 (segment (start 124.37 61) (end 133.16 61) (width 1) (layer "F.Cu") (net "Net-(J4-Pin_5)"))
 (segment (start 124.285 61.085) (end 124.37 61) (width 1) (layer "F.Cu") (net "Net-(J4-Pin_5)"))
 (segment (start 133.16 61) (end 133.5 60.66) (width 1) (layer "F.Cu") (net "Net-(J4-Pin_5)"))
 (segment (start 133.195 63.505) (end 133.5 63.2) (width 1) (layer "F.Cu") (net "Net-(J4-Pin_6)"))
 (segment (start 124.315 63.505) (end 133.195 63.505) (width 1) (layer "F.Cu") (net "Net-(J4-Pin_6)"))
 (segment (start 66 78.5) (end 66 77) (width 1) (layer "F.Cu") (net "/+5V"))
 (segment (start 66 77) (end 66 58.38) (width 1) (layer "F.Cu") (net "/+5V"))
 (segment (start 78.45 94.43) (end 78.45 94.05) (width 1) (layer "F.Cu") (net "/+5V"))
 (segment (start 78.5 91) (end 66 78.5) (width 1) (layer "F.Cu") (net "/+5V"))
 (segment (start 78.45 94.05) (end 78.5 94) (width 1) (layer "F.Cu") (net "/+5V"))
 (segment (start 78.5 94) (end 78.5 91) (width 1) (layer "F.Cu") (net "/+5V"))
 (segment (start 95 62.43) (end 95 62.5) (width 1) (layer "F.Cu") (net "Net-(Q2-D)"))
 (segment (start 98.315 61.085) (end 96.345 61.085) (width 1) (layer "F.Cu") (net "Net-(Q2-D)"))
 (segment (start 96.345 61.085) (end 95 62.43) (width 1) (layer "F.Cu") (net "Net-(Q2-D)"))
 (segment (start 92.5 65) (end 89 65) (width 1) (layer "F.Cu") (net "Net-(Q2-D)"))
 (segment (start 95 62.5) (end 92.5 65) (width 1) (layer "F.Cu") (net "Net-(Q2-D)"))
 (segment (start 125 69) (end 122 66) (width 1) (layer "F.Cu") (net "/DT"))
 (segment (start 111.5 66) (end 101.505 56.005) (width 1) (layer "F.Cu") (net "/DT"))
 (segment (start 122 66) (end 111.5 66) (width 1) (layer "F.Cu") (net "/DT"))
 (segment (start 101.505 56.005) (end 98.315 56.005) (width 1) (layer "F.Cu") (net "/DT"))
 (segment (start 116.55 94.43) (end 125 85.98) (width 1) (layer "F.Cu") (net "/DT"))
 (segment (start 125 85.98) (end 125 69) (width 1) (layer "F.Cu") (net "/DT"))
 (segment (start 122 83.5) (end 122 70.5) (width 1) (layer "F.Cu") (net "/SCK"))
 (segment (start 101.31 94.43) (end 104.74 91) (width 1) (layer "F.Cu") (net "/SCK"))
 (segment (start 114.5 91) (end 122 83.5) (width 1) (layer "F.Cu") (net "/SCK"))
 (segment (start 122 70.5) (end 120 68.5) (width 1) (layer "F.Cu") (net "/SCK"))
 (segment (start 100 58.5) (end 98.5 58.5) (width 1) (layer "F.Cu") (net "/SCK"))
 (segment (start 110 68.5) (end 100 58.5) (width 1) (layer "F.Cu") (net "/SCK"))
 (segment (start 120 68.5) (end 110 68.5) (width 1) (layer "F.Cu") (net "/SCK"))
 (segment (start 104.74 91) (end 114.5 91) (width 1) (layer "F.Cu") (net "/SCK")))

